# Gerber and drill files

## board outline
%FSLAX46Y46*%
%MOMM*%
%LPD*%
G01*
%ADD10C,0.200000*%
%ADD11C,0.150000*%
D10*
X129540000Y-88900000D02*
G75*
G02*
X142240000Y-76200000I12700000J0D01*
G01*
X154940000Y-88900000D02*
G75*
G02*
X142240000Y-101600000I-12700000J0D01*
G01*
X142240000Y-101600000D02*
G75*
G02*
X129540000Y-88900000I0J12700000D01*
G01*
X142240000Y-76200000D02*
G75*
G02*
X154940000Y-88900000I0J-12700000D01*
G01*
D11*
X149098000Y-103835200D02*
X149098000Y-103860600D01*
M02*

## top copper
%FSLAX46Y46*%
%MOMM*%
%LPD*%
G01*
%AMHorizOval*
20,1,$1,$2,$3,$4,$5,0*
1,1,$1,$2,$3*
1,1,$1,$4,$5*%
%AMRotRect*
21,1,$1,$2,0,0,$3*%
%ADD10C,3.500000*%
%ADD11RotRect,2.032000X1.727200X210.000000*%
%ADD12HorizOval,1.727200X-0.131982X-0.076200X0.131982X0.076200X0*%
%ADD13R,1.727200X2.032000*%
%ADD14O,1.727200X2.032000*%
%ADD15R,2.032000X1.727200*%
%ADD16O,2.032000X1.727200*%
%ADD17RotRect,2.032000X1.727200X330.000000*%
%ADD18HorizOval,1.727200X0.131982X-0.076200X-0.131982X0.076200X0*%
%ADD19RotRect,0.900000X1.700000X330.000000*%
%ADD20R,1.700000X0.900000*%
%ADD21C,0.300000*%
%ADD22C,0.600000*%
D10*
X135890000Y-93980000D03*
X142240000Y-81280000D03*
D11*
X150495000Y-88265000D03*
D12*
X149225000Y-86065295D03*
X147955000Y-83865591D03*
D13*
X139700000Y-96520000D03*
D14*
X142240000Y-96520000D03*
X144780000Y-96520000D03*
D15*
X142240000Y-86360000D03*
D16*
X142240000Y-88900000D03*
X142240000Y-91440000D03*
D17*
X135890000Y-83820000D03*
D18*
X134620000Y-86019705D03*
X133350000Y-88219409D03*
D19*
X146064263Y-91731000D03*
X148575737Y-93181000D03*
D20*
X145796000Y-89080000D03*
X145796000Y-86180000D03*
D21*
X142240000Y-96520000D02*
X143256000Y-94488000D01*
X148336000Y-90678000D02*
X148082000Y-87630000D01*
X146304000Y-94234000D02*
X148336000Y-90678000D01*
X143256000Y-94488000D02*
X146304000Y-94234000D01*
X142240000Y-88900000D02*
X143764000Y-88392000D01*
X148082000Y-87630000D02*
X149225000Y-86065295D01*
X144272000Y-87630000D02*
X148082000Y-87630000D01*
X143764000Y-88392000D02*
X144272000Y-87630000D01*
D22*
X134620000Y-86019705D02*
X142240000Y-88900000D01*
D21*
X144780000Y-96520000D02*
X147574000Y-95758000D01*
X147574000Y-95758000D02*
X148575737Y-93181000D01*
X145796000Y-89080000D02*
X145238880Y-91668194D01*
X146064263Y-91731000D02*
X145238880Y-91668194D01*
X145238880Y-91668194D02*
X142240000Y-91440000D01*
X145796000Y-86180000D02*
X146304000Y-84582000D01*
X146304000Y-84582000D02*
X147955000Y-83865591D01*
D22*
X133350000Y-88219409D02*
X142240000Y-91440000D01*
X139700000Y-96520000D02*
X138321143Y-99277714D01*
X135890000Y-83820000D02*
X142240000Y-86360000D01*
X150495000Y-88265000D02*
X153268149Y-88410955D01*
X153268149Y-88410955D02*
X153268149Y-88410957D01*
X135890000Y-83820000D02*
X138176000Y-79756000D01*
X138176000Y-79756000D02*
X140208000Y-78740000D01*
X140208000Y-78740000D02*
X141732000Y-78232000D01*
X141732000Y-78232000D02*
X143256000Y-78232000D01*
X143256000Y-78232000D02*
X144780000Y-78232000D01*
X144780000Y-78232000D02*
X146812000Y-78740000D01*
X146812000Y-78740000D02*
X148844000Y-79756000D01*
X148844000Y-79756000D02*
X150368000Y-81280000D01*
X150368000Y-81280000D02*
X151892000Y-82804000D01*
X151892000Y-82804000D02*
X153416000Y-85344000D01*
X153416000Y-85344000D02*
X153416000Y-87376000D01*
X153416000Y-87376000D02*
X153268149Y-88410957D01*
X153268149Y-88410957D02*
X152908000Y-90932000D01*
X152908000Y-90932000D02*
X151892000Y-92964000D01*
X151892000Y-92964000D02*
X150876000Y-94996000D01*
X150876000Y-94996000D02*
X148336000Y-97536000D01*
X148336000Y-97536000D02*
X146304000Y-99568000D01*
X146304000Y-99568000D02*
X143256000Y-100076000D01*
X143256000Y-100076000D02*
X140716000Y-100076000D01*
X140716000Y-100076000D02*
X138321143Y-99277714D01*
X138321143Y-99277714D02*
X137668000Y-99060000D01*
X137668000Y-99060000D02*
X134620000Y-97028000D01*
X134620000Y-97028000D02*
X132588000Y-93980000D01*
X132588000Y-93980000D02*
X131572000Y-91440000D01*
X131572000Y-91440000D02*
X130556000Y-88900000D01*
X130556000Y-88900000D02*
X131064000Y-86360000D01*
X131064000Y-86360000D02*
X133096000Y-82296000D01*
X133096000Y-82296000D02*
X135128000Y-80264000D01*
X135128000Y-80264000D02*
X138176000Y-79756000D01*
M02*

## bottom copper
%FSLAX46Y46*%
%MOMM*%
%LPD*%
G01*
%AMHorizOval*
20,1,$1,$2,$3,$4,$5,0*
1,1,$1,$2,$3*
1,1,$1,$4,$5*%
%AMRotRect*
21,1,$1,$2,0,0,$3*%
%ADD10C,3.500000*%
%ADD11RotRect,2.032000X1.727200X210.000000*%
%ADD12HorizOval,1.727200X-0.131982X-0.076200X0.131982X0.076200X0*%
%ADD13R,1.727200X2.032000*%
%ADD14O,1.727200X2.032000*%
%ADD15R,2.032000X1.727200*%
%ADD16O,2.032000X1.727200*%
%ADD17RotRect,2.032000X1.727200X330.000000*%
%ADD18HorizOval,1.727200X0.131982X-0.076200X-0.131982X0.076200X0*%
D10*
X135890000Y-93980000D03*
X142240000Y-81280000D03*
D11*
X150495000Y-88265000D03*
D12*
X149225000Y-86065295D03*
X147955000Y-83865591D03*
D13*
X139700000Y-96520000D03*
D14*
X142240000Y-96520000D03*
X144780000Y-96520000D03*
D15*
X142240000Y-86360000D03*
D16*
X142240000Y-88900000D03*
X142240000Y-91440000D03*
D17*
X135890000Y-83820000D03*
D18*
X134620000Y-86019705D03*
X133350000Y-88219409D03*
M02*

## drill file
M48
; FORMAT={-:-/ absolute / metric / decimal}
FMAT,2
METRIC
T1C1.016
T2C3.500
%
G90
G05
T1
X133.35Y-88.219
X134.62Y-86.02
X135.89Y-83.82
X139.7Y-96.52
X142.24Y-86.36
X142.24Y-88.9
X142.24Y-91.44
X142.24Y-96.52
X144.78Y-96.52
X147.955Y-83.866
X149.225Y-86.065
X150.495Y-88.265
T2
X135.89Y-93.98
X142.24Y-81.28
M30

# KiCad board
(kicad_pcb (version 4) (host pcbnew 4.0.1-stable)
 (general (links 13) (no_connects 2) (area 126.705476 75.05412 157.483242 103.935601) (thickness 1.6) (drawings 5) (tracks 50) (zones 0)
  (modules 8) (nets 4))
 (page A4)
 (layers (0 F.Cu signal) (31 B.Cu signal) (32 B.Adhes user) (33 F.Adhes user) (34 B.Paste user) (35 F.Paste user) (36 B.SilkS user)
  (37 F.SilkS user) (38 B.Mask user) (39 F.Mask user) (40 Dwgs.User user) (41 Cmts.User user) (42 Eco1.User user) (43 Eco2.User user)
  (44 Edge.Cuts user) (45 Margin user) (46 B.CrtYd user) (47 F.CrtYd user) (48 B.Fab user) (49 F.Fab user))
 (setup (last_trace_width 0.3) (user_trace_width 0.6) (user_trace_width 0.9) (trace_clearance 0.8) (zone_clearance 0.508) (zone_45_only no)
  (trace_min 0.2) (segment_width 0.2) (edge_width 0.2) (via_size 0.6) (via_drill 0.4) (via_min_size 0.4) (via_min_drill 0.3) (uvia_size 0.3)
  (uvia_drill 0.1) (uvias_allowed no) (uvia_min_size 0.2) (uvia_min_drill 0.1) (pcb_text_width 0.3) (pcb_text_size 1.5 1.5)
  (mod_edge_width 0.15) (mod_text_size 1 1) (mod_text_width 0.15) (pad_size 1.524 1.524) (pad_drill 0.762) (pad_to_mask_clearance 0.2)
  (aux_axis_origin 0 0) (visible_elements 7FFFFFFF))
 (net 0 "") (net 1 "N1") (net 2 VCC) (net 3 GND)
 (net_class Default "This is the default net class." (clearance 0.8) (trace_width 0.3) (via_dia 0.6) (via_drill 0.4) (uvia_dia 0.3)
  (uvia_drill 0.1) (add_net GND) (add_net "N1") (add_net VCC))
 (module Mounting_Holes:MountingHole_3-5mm (layer F.Cu) (at 135.89 93.98)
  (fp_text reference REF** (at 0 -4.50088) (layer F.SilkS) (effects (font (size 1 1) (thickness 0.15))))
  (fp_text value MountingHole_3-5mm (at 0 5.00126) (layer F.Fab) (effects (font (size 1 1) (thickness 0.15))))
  (pad 1 thru_hole circle (at 0 0) (size 3.5 3.5) (drill 3.5) (layers)))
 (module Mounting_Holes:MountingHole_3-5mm (layer F.Cu) (at 142.24 81.28)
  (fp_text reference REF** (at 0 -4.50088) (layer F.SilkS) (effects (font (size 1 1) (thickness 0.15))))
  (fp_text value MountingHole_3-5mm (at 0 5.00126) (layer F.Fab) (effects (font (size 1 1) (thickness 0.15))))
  (pad 1 thru_hole circle (at 0 0) (size 3.5 3.5) (drill 3.5) (layers)))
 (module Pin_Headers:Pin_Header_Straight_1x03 (layer F.Cu) (at 150.495 88.265 210)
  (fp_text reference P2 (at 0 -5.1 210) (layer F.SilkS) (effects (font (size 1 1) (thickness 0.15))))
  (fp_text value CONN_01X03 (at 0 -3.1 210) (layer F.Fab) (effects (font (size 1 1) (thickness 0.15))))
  (pad 1 thru_hole rect (at 0 0 210) (size 2.032 1.7272) (drill 1.016) (layers *.Cu *.Mask) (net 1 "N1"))
  (pad 2 thru_hole oval (at 0 2.54 210) (size 2.032 1.7272) (drill 1.016) (layers *.Cu *.Mask) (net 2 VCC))
  (pad 3 thru_hole oval (at 0 5.08 210) (size 2.032 1.7272) (drill 1.016) (layers *.Cu *.Mask) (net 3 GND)))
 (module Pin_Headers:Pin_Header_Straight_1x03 (layer F.Cu) (at 139.7 96.52 90)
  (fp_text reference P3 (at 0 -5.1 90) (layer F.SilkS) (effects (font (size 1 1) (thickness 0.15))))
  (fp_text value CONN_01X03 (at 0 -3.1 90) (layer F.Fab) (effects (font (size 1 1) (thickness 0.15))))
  (pad 1 thru_hole rect (at 0 0 90) (size 2.032 1.7272) (drill 1.016) (layers *.Cu *.Mask) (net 1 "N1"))
  (pad 2 thru_hole oval (at 0 2.54 90) (size 2.032 1.7272) (drill 1.016) (layers *.Cu *.Mask) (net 2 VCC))
  (pad 3 thru_hole oval (at 0 5.08 90) (size 2.032 1.7272) (drill 1.016) (layers *.Cu *.Mask) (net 3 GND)))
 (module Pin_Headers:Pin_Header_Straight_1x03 (layer F.Cu) (at 142.24 86.36)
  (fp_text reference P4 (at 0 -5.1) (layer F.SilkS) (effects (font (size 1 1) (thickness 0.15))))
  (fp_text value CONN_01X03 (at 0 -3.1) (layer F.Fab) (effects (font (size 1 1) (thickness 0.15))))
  (pad 1 thru_hole rect (at 0 0) (size 2.032 1.7272) (drill 1.016) (layers *.Cu *.Mask) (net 1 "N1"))
  (pad 2 thru_hole oval (at 0 2.54) (size 2.032 1.7272) (drill 1.016) (layers *.Cu *.Mask) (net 2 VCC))
  (pad 3 thru_hole oval (at 0 5.08) (size 2.032 1.7272) (drill 1.016) (layers *.Cu *.Mask) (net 3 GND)))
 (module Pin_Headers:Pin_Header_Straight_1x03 (layer F.Cu) (at 135.89 83.82 330)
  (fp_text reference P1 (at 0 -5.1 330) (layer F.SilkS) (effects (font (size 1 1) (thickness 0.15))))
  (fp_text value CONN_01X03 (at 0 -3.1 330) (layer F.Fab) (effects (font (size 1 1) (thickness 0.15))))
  (pad 1 thru_hole rect (at 0 0 330) (size 2.032 1.7272) (drill 1.016) (layers *.Cu *.Mask) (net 1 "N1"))
  (pad 2 thru_hole oval (at 0 2.54 330) (size 2.032 1.7272) (drill 1.016) (layers *.Cu *.Mask) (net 2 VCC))
  (pad 3 thru_hole oval (at 0 5.08 330) (size 2.032 1.7272) (drill 1.016) (layers *.Cu *.Mask) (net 3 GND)))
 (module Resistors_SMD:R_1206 (layer F.Cu) (at 147.32 92.456 330)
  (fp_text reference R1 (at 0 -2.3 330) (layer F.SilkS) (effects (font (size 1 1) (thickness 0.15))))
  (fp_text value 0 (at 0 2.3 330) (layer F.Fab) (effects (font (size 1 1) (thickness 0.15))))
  (pad 1 smd rect (at -1.45 0 330) (size 0.9 1.7) (layers F.Cu F.Paste F.Mask) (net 3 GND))
  (pad 2 smd rect (at 1.45 0 330) (size 0.9 1.7) (layers F.Cu F.Paste F.Mask) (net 3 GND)))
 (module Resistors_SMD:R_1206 (layer F.Cu) (at 145.796 87.63 90)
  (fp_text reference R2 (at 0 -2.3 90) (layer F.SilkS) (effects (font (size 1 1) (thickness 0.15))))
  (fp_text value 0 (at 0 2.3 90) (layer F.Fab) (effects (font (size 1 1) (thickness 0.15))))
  (pad 1 smd rect (at -1.45 0 90) (size 0.9 1.7) (layers F.Cu F.Paste F.Mask) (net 3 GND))
  (pad 2 smd rect (at 1.45 0 90) (size 0.9 1.7) (layers F.Cu F.Paste F.Mask) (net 3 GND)))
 (gr_arc (start 142.24 88.9) (end 129.54 88.9) (angle 90) (layer Edge.Cuts) (width 0.2))
 (gr_arc (start 142.24 88.9) (end 154.94 88.9) (angle 90) (layer Edge.Cuts) (width 0.2))
 (gr_arc (start 142.24 88.9) (end 142.24 101.6) (angle 90) (layer Edge.Cuts) (width 0.2))
 (gr_arc (start 142.24 88.9) (end 142.24 76.2) (angle 90) (layer Edge.Cuts) (width 0.2))
 (gr_line (start 149.098 103.8352) (end 149.098 103.8606) (angle 90) (layer Edge.Cuts) (width 0.15))
 (segment (start 142.24 96.52) (end 143.256 94.488) (width 0.3) (layer F.Cu) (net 2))
 (segment (start 148.336 90.678) (end 148.082 87.63) (width 0.3) (layer F.Cu) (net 2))
 (segment (start 146.304 94.234) (end 148.336 90.678) (width 0.3) (layer F.Cu) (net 2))
 (segment (start 143.256 94.488) (end 146.304 94.234) (width 0.3) (layer F.Cu) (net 2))
 (segment (start 142.24 88.9) (end 143.764 88.392) (width 0.3) (layer F.Cu) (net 2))
 (segment (start 148.082 87.63) (end 149.225 86.065295) (width 0.3) (layer F.Cu) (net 2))
 (segment (start 144.272 87.63) (end 148.082 87.63) (width 0.3) (layer F.Cu) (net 2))
 (segment (start 143.764 88.392) (end 144.272 87.63) (width 0.3) (layer F.Cu) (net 2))
 (segment (start 134.62 86.019705) (end 142.24 88.9) (width 0.6) (layer F.Cu) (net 2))
 (segment (start 144.78 96.52) (end 147.574 95.758) (width 0.3) (layer F.Cu) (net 3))
 (segment (start 147.574 95.758) (end 148.575737 93.181) (width 0.3) (layer F.Cu) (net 3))
 (segment (start 145.796 89.08) (end 145.23888 91.668194) (width 0.3) (layer F.Cu) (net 3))
 (segment (start 146.064263 91.731) (end 145.23888 91.668194) (width 0.3) (layer F.Cu) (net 3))
 (segment (start 145.23888 91.668194) (end 142.24 91.44) (width 0.3) (layer F.Cu) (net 3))
 (segment (start 145.796 86.18) (end 146.304 84.582) (width 0.3) (layer F.Cu) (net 3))
 (segment (start 146.304 84.582) (end 147.955 83.865591) (width 0.3) (layer F.Cu) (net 3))
 (segment (start 133.35 88.219409) (end 142.24 91.44) (width 0.6) (layer F.Cu) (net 3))
 (segment (start 139.7 96.52) (end 138.321143 99.277714) (width 0.6) (layer F.Cu) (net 1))
 (segment (start 135.89 83.82) (end 142.24 86.36) (width 0.6) (layer F.Cu) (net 1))
 (segment (start 150.495 88.265) (end 153.268149 88.410955) (width 0.6) (layer F.Cu) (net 1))
 (segment (start 153.268149 88.410955) (end 153.268149 88.410957) (width 0.6) (layer F.Cu) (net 1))
 (segment (start 135.89 83.82) (end 138.176 79.756) (width 0.6) (layer F.Cu) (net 1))
 (segment (start 138.176 79.756) (end 140.208 78.74) (width 0.6) (layer F.Cu) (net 1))
 (segment (start 140.208 78.74) (end 141.732 78.232) (width 0.6) (layer F.Cu) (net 1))
 (segment (start 141.732 78.232) (end 143.256 78.232) (width 0.6) (layer F.Cu) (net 1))
 (segment (start 143.256 78.232) (end 144.78 78.232) (width 0.6) (layer F.Cu) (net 1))
 (segment (start 144.78 78.232) (end 146.812 78.74) (width 0.6) (layer F.Cu) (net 1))
 (segment (start 146.812 78.74) (end 148.844 79.756) (width 0.6) (layer F.Cu) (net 1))
 (segment (start 148.844 79.756) (end 150.368 81.28) (width 0.6) (layer F.Cu) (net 1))
 (segment (start 150.368 81.28) (end 151.892 82.804) (width 0.6) (layer F.Cu) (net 1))
 (segment (start 151.892 82.804) (end 153.416 85.344) (width 0.6) (layer F.Cu) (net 1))
 (segment (start 153.416 85.344) (end 153.416 87.376) (width 0.6) (layer F.Cu) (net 1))
 (segment (start 153.416 87.376) (end 153.268149 88.410957) (width 0.6) (layer F.Cu) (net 1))
 (segment (start 153.268149 88.410957) (end 152.908 90.932) (width 0.6) (layer F.Cu) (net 1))
 (segment (start 152.908 90.932) (end 151.892 92.964) (width 0.6) (layer F.Cu) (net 1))
 (segment (start 151.892 92.964) (end 150.876 94.996) (width 0.6) (layer F.Cu) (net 1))
 (segment (start 150.876 94.996) (end 148.336 97.536) (width 0.6) (layer F.Cu) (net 1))
 (segment (start 148.336 97.536) (end 146.304 99.568) (width 0.6) (layer F.Cu) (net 1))
 (segment (start 146.304 99.568) (end 143.256 100.076) (width 0.6) (layer F.Cu) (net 1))
 (segment (start 143.256 100.076) (end 140.716 100.076) (width 0.6) (layer F.Cu) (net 1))
 (segment (start 140.716 100.076) (end 138.321143 99.277714) (width 0.6) (layer F.Cu) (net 1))
 (segment (start 138.321143 99.277714) (end 137.668 99.06) (width 0.6) (layer F.Cu) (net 1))
 (segment (start 137.668 99.06) (end 134.62 97.028) (width 0.6) (layer F.Cu) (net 1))
 (segment (start 134.62 97.028) (end 132.588 93.98) (width 0.6) (layer F.Cu) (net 1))
 (segment (start 132.588 93.98) (end 131.572 91.44) (width 0.6) (layer F.Cu) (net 1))
 (segment (start 131.572 91.44) (end 130.556 88.9) (width 0.6) (layer F.Cu) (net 1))
 (segment (start 130.556 88.9) (end 131.064 86.36) (width 0.6) (layer F.Cu) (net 1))
 (segment (start 131.064 86.36) (end 133.096 82.296) (width 0.6) (layer F.Cu) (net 1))
 (segment (start 133.096 82.296) (end 135.128 80.264) (width 0.6) (layer F.Cu) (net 1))
 (segment (start 135.128 80.264) (end 138.176 79.756) (width 0.6) (layer F.Cu) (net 1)))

